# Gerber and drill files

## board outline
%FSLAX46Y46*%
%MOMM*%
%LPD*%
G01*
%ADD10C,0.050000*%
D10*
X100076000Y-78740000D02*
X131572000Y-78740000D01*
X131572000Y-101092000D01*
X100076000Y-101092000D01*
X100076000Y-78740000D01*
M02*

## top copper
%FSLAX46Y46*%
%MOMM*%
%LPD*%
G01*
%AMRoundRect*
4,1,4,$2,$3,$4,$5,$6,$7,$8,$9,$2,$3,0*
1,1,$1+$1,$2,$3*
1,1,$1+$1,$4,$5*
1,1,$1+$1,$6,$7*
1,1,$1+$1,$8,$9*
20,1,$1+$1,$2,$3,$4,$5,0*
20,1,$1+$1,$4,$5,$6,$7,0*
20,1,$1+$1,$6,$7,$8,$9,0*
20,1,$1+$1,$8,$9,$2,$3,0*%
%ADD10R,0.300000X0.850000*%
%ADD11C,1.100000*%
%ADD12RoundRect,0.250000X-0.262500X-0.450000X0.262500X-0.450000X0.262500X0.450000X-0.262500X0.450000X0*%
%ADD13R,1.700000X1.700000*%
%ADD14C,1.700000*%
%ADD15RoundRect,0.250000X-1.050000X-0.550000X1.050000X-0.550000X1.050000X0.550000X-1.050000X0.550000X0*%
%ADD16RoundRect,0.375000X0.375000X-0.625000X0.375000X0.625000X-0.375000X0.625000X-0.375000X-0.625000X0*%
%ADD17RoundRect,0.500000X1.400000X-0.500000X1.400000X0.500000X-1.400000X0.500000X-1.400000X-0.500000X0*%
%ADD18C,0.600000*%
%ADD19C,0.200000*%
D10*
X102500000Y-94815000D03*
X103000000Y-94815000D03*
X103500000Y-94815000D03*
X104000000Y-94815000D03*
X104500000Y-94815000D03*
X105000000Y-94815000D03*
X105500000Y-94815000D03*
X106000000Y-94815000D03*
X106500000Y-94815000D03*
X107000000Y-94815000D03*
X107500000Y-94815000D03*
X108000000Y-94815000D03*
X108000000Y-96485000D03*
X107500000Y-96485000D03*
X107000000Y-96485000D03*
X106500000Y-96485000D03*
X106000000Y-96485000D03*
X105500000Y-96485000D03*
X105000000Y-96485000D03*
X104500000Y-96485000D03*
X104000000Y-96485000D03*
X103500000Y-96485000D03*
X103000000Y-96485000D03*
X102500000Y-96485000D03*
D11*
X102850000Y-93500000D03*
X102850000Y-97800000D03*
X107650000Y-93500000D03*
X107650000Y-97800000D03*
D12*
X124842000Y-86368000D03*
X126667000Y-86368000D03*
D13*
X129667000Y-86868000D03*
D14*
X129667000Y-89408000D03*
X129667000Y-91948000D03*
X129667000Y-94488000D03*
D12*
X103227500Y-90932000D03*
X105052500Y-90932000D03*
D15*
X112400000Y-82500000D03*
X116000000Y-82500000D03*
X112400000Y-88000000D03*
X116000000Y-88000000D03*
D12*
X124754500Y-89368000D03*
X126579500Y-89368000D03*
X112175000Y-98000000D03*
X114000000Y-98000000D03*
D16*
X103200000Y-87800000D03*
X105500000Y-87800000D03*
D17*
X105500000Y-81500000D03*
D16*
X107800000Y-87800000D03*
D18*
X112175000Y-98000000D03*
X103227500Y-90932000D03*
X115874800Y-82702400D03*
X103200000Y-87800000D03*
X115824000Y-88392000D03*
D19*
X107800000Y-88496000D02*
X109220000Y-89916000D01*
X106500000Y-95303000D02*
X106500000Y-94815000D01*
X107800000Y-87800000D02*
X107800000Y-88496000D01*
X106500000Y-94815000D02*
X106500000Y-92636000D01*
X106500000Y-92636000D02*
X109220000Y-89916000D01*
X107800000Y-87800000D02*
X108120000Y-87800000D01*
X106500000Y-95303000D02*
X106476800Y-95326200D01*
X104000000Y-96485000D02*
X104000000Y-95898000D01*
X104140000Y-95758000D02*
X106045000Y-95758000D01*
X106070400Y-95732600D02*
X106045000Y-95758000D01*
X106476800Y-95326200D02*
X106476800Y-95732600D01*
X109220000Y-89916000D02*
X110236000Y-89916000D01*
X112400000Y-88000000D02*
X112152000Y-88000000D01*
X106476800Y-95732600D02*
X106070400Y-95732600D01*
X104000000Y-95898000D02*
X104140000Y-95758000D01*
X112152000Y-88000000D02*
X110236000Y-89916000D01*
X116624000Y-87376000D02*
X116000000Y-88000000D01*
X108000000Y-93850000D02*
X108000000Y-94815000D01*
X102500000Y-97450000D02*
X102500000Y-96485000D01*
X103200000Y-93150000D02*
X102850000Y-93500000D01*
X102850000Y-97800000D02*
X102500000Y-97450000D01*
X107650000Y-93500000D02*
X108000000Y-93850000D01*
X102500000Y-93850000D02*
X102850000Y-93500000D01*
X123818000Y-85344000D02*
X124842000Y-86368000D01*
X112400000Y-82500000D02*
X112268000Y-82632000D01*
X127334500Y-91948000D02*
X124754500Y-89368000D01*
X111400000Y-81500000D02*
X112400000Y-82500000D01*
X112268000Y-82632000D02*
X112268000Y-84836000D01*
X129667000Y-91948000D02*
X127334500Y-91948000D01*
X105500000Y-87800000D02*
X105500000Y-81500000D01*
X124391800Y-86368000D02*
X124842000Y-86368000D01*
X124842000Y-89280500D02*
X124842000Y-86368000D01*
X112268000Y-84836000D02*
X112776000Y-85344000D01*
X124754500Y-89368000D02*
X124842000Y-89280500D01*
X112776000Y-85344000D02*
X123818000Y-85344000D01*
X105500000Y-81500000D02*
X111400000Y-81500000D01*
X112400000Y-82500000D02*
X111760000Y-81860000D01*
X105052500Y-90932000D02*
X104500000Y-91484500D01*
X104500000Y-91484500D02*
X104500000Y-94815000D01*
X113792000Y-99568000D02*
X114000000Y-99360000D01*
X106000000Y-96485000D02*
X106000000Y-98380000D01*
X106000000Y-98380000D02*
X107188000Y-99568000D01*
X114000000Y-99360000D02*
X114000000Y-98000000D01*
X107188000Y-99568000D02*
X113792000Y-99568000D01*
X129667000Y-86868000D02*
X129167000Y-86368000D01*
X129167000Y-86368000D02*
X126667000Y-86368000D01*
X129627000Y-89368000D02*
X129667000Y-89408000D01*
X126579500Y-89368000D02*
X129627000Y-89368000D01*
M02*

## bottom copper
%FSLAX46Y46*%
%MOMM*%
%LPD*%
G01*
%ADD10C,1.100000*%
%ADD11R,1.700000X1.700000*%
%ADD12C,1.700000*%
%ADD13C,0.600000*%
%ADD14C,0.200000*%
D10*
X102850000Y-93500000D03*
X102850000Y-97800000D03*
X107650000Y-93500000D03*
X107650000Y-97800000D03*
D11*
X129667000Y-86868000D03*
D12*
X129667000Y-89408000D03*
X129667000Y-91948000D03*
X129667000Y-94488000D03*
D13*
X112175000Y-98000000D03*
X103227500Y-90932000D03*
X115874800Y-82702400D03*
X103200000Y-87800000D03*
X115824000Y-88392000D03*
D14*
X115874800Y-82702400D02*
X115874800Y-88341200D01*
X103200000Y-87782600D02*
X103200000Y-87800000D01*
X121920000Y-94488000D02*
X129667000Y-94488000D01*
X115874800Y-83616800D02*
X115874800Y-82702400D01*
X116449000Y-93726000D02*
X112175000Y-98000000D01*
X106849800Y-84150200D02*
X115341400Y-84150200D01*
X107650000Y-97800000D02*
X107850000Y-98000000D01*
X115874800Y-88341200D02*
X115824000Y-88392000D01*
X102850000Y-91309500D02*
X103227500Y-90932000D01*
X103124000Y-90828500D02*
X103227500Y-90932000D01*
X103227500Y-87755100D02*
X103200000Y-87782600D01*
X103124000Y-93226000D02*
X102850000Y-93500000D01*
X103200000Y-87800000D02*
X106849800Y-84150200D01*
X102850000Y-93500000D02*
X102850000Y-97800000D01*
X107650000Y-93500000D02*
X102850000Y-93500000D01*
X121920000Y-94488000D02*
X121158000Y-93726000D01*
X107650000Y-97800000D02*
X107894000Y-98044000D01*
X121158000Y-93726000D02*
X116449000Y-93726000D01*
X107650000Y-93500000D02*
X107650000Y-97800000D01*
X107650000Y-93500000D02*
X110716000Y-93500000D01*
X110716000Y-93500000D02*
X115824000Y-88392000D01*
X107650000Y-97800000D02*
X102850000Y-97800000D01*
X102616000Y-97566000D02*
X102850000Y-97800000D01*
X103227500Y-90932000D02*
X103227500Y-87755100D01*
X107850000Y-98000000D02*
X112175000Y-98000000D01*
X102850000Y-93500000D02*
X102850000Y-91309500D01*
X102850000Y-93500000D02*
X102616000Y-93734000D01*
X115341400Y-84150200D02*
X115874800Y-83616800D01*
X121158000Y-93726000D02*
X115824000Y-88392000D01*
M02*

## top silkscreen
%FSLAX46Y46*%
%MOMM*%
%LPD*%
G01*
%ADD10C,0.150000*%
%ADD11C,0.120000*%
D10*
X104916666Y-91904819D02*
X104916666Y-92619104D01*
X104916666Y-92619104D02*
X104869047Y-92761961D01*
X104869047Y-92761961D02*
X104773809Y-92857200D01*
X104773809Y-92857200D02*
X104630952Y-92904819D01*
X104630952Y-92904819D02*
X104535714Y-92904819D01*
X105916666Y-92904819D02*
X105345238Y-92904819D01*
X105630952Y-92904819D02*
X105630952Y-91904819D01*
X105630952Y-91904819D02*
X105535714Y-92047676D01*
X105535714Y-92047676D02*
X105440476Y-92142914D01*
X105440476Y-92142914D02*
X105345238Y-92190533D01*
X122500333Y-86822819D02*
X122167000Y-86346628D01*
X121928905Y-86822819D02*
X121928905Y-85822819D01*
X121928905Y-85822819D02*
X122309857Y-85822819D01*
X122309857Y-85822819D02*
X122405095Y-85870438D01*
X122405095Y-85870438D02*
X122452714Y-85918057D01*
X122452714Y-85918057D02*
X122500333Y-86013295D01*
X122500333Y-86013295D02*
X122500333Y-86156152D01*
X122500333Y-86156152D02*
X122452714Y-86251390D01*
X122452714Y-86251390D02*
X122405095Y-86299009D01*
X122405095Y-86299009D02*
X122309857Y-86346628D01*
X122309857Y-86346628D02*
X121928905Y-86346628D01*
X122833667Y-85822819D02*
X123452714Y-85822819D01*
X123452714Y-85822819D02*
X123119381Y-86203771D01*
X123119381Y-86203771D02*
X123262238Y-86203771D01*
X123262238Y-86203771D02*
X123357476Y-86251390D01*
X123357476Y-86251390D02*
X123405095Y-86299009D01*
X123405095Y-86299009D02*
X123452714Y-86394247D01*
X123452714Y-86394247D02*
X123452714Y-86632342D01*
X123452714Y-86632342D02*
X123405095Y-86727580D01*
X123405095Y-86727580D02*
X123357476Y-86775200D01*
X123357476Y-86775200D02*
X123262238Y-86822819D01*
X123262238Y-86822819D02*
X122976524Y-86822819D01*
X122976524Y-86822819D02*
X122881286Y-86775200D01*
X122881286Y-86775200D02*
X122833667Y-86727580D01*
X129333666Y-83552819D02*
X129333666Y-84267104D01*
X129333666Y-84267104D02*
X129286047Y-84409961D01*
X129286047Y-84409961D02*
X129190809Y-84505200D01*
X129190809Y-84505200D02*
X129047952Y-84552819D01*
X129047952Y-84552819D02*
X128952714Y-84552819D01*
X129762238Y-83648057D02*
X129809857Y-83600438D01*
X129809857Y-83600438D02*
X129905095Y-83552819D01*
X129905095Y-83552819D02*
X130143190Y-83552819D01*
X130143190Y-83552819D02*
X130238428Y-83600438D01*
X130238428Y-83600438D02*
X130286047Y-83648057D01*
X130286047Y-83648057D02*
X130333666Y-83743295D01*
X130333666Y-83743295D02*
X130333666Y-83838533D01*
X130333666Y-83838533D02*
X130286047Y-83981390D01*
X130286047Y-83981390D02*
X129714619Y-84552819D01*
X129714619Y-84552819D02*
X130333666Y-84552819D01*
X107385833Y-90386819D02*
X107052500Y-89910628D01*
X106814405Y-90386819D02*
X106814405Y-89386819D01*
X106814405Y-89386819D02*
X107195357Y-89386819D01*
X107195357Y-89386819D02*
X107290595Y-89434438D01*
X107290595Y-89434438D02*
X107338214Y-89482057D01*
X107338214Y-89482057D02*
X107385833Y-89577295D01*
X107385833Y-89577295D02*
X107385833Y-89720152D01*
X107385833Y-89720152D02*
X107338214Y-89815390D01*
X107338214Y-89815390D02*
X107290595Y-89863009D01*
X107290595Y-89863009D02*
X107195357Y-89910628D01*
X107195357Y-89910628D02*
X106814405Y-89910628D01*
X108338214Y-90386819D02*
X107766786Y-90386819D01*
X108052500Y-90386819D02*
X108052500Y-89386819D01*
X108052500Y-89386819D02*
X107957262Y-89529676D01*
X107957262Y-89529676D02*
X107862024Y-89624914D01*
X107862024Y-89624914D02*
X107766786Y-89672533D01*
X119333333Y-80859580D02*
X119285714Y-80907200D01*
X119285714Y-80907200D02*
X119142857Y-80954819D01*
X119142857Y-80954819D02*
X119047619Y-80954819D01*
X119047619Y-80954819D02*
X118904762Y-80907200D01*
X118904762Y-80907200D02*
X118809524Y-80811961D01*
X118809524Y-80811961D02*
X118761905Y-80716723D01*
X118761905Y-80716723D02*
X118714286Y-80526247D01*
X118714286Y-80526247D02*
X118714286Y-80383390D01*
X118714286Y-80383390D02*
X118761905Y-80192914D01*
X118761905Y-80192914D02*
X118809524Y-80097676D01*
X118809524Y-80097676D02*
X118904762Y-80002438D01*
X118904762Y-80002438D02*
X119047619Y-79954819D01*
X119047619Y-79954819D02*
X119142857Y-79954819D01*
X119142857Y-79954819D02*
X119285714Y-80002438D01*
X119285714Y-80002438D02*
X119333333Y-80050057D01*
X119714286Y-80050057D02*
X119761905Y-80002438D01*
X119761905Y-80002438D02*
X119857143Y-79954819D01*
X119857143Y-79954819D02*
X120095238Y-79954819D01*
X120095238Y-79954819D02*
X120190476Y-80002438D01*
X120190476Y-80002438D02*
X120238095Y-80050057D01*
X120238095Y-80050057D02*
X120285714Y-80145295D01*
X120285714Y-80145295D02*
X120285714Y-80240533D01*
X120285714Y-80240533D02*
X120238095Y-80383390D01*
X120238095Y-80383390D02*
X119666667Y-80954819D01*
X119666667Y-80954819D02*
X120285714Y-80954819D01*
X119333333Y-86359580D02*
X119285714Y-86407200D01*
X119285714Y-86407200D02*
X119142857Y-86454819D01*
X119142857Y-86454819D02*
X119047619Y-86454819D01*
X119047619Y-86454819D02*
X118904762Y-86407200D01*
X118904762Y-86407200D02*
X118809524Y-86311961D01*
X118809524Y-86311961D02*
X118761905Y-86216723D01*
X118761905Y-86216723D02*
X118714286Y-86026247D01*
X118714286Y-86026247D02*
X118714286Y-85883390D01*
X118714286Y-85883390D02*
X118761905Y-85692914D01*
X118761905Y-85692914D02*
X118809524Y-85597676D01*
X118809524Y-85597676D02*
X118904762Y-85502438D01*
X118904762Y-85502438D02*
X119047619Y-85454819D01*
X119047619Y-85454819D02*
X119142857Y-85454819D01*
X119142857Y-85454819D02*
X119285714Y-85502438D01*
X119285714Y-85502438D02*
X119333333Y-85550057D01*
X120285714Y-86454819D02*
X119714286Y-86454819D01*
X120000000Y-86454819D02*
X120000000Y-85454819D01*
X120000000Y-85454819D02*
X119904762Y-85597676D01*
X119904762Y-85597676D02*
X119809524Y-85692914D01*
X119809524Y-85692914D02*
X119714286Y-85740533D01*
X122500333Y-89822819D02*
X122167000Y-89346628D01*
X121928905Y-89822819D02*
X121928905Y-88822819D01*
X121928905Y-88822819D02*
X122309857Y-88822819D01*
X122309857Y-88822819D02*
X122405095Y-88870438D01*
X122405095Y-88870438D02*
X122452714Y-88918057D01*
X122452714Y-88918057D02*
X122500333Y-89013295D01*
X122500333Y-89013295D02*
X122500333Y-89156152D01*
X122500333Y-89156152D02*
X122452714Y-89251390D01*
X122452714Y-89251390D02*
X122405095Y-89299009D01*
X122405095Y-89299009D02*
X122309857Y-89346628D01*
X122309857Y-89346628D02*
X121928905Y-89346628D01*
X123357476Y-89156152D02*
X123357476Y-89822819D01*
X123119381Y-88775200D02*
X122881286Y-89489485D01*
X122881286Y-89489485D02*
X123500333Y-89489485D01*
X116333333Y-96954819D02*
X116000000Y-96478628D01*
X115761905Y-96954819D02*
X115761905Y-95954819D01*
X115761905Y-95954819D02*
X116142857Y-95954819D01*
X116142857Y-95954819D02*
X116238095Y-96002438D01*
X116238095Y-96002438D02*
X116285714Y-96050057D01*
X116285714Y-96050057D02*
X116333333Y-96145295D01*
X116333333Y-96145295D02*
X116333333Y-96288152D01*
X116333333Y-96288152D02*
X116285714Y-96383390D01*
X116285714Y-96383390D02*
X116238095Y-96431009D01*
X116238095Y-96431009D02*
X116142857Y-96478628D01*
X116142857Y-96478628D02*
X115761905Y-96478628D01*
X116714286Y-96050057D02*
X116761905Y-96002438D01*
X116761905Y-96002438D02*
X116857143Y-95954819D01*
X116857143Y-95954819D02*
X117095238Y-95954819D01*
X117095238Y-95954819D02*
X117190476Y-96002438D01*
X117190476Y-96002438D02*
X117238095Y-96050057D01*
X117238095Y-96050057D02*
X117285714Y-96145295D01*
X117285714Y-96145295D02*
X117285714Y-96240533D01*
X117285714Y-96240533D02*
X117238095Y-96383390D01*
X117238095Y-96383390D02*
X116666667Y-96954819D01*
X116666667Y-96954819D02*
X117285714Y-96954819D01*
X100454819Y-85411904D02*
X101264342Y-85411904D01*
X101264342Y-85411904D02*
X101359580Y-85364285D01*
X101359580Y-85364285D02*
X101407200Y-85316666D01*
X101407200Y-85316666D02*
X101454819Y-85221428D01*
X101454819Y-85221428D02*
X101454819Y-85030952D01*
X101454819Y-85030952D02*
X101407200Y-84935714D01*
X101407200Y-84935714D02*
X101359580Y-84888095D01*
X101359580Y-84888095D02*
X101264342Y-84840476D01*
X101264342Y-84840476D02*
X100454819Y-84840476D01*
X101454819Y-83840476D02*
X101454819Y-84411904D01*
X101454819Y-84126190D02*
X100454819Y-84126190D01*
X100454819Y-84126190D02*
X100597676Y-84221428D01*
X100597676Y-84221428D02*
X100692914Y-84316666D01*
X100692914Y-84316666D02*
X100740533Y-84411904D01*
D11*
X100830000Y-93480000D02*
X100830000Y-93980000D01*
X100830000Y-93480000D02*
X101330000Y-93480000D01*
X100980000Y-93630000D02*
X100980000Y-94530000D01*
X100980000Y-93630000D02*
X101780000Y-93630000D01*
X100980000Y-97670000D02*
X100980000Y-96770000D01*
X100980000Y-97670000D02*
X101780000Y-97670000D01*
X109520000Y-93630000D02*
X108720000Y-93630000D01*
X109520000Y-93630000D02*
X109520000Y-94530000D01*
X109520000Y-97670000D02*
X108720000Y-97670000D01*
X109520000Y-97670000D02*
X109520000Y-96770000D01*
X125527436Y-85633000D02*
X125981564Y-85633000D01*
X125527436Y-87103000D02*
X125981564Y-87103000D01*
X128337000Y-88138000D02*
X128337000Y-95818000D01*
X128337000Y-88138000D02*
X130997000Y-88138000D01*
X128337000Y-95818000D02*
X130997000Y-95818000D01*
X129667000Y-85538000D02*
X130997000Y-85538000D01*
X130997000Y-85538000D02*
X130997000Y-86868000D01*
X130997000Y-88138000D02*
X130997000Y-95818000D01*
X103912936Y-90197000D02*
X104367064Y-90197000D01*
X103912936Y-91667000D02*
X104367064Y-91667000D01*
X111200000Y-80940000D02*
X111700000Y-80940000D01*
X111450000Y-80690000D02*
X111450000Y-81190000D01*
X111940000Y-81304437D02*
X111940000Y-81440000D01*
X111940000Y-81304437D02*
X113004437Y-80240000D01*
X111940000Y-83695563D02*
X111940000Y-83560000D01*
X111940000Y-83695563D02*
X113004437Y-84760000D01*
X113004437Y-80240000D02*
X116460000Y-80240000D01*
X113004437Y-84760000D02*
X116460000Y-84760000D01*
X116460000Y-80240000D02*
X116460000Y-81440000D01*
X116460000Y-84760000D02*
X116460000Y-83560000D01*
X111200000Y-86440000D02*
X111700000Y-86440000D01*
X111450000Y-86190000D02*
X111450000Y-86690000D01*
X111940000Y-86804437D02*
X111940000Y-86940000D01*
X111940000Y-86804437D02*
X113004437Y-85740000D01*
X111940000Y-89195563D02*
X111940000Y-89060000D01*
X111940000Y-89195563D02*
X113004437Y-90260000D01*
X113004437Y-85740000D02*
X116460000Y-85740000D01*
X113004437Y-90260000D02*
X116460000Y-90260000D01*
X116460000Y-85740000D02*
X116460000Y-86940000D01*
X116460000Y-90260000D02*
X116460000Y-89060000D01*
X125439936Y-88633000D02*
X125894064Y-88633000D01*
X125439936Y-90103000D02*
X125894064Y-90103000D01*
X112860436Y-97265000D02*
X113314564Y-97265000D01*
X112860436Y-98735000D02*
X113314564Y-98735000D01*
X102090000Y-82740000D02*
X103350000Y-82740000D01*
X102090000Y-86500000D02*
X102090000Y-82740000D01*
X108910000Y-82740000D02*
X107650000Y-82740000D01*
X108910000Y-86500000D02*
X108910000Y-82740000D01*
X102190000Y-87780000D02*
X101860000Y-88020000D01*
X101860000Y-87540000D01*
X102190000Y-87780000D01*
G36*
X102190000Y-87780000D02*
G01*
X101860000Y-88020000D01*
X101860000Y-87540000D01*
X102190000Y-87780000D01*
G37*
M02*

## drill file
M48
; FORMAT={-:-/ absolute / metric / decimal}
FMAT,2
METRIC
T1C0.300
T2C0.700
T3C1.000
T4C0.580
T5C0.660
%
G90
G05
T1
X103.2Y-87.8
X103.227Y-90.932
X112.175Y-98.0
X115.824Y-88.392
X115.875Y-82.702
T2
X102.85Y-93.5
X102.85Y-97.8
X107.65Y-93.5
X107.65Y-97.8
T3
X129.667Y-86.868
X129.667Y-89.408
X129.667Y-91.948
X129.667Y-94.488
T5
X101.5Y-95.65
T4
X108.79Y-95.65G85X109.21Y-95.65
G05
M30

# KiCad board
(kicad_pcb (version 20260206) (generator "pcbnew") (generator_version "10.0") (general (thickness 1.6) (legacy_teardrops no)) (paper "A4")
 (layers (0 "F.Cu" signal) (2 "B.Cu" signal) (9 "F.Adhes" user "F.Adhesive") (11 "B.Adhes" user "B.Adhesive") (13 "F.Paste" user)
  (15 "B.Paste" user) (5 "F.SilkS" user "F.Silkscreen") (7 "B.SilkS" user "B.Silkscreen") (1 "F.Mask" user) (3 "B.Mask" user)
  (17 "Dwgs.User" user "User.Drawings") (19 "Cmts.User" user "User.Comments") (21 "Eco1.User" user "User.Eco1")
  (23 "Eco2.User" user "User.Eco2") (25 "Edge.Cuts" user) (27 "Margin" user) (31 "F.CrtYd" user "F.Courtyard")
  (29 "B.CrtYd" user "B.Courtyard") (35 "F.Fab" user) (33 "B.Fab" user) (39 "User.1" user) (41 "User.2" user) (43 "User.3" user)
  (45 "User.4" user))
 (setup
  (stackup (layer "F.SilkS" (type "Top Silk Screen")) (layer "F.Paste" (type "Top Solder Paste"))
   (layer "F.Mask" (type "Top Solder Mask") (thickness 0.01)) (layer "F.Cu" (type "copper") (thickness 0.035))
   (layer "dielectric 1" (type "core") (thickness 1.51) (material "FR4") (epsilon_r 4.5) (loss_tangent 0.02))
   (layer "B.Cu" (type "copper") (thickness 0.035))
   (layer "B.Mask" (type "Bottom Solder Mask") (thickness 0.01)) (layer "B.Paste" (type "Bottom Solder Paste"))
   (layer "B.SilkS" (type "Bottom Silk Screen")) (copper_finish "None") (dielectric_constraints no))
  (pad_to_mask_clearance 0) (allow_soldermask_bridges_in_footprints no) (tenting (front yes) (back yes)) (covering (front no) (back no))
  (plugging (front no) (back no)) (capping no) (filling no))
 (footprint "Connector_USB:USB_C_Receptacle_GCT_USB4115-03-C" (layer "F.Cu") (at 105.25 95.65)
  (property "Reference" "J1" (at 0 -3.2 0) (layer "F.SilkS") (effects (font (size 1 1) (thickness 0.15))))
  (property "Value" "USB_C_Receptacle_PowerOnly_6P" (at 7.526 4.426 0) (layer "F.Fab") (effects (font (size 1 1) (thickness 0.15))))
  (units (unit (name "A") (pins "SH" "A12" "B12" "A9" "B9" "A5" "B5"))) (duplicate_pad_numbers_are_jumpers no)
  (fp_line (start -4.42 -2.17) (end -4.42 -1.67) (stroke (width 0.12) (type solid)) (layer "F.SilkS"))
  (fp_line (start -4.42 -2.17) (end -3.92 -2.17) (stroke (width 0.12) (type solid)) (layer "F.SilkS"))
  (fp_line (start -4.27 -2.02) (end -4.27 -1.12) (stroke (width 0.12) (type solid)) (layer "F.SilkS"))
  (fp_line (start -4.27 -2.02) (end -3.47 -2.02) (stroke (width 0.12) (type solid)) (layer "F.SilkS"))
  (fp_line (start -4.27 2.02) (end -4.27 1.12) (stroke (width 0.12) (type solid)) (layer "F.SilkS"))
  (fp_line (start -4.27 2.02) (end -3.47 2.02) (stroke (width 0.12) (type solid)) (layer "F.SilkS"))
  (fp_line (start 4.27 -2.02) (end 3.47 -2.02) (stroke (width 0.12) (type solid)) (layer "F.SilkS"))
  (fp_line (start 4.27 -2.02) (end 4.27 -1.12) (stroke (width 0.12) (type solid)) (layer "F.SilkS"))
  (fp_line (start 4.27 2.02) (end 3.47 2.02) (stroke (width 0.12) (type solid)) (layer "F.SilkS"))
  (fp_line (start 4.27 2.02) (end 4.27 1.12) (stroke (width 0.12) (type solid)) (layer "F.SilkS"))
  (pad "" np_thru_hole circle (at -3.75 0) (size 0.66 0.66) (drill 0.66) (layers "*.Cu" "*.Mask"))
  (pad "" np_thru_hole oval (at 3.75 0) (size 1 0.58) (drill oval 1 0.58) (layers "*.Cu" "*.Mask"))
  (pad "A1" smd rect (at -2.75 -0.835) (size 0.3 0.85) (layers "F.Cu" "F.Mask" "F.Paste"))
  (pad "A2" smd rect (at -2.25 -0.835) (size 0.3 0.85) (layers "F.Cu" "F.Mask" "F.Paste"))
  (pad "A3" smd rect (at -1.75 -0.835) (size 0.3 0.85) (layers "F.Cu" "F.Mask" "F.Paste"))
  (pad "A4" smd rect (at -1.25 -0.835) (size 0.3 0.85) (layers "F.Cu" "F.Mask" "F.Paste"))
  (pad "A5" smd rect (at -0.75 -0.835) (size 0.3 0.85) (layers "F.Cu" "F.Mask" "F.Paste") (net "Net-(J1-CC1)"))
  (pad "A6" smd rect (at -0.25 -0.835) (size 0.3 0.85) (layers "F.Cu" "F.Mask" "F.Paste"))
  (pad "A7" smd rect (at 0.25 -0.835) (size 0.3 0.85) (layers "F.Cu" "F.Mask" "F.Paste"))
  (pad "A8" smd rect (at 0.75 -0.835) (size 0.3 0.85) (layers "F.Cu" "F.Mask" "F.Paste"))
  (pad "A9" smd rect (at 1.25 -0.835) (size 0.3 0.85) (layers "F.Cu" "F.Mask" "F.Paste") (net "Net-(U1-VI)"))
  (pad "A10" smd rect (at 1.75 -0.835) (size 0.3 0.85) (layers "F.Cu" "F.Mask" "F.Paste"))
  (pad "A11" smd rect (at 2.25 -0.835) (size 0.3 0.85) (layers "F.Cu" "F.Mask" "F.Paste"))
  (pad "A12" smd rect (at 2.75 -0.835) (size 0.3 0.85) (layers "F.Cu" "F.Mask" "F.Paste") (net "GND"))
  (pad "B1" smd rect (at 2.75 0.835) (size 0.3 0.85) (layers "F.Cu" "F.Mask" "F.Paste"))
  (pad "B2" smd rect (at 2.25 0.835) (size 0.3 0.85) (layers "F.Cu" "F.Mask" "F.Paste"))
  (pad "B3" smd rect (at 1.75 0.835) (size 0.3 0.85) (layers "F.Cu" "F.Mask" "F.Paste"))
  (pad "B4" smd rect (at 1.25 0.835) (size 0.3 0.85) (layers "F.Cu" "F.Mask" "F.Paste"))
  (pad "B5" smd rect (at 0.75 0.835) (size 0.3 0.85) (layers "F.Cu" "F.Mask" "F.Paste") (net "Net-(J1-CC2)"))
  (pad "B6" smd rect (at 0.25 0.835) (size 0.3 0.85) (layers "F.Cu" "F.Mask" "F.Paste"))
  (pad "B7" smd rect (at -0.25 0.835) (size 0.3 0.85) (layers "F.Cu" "F.Mask" "F.Paste"))
  (pad "B8" smd rect (at -0.75 0.835) (size 0.3 0.85) (layers "F.Cu" "F.Mask" "F.Paste"))
  (pad "B9" smd rect (at -1.25 0.835) (size 0.3 0.85) (layers "F.Cu" "F.Mask" "F.Paste") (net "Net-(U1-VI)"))
  (pad "B10" smd rect (at -1.75 0.835) (size 0.3 0.85) (layers "F.Cu" "F.Mask" "F.Paste"))
  (pad "B11" smd rect (at -2.25 0.835) (size 0.3 0.85) (layers "F.Cu" "F.Mask" "F.Paste"))
  (pad "B12" smd rect (at -2.75 0.835) (size 0.3 0.85) (layers "F.Cu" "F.Mask" "F.Paste") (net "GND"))
  (pad "SH" thru_hole circle (at -2.4 -2.15) (size 1.1 1.1) (drill 0.7) (layers "*.Cu" "*.Mask" "F.Paste") (remove_unused_layers no)
   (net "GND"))
  (pad "SH" thru_hole circle (at -2.4 2.15) (size 1.1 1.1) (drill 0.7) (layers "*.Cu" "*.Mask" "F.Paste") (remove_unused_layers no)
   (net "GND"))
  (pad "SH" thru_hole circle (at 2.4 -2.15) (size 1.1 1.1) (drill 0.7) (layers "*.Cu" "*.Mask" "F.Paste") (remove_unused_layers no)
   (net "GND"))
  (pad "SH" thru_hole circle (at 2.4 2.15) (size 1.1 1.1) (drill 0.7) (layers "*.Cu" "*.Mask" "F.Paste") (remove_unused_layers no)
   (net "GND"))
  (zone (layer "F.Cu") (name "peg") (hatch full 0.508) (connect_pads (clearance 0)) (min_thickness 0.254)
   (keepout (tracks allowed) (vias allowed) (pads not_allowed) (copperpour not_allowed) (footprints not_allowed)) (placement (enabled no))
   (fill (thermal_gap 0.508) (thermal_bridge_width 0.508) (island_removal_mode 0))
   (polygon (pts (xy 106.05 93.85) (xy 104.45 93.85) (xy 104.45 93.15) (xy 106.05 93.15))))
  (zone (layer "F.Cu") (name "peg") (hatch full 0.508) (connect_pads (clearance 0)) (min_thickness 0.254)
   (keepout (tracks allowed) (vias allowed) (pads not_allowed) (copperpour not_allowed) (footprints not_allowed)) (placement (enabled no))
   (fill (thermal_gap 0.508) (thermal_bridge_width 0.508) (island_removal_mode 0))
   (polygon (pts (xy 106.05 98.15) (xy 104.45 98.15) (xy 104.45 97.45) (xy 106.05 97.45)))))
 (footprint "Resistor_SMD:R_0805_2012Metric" (layer "F.Cu") (at 125.7545 86.368)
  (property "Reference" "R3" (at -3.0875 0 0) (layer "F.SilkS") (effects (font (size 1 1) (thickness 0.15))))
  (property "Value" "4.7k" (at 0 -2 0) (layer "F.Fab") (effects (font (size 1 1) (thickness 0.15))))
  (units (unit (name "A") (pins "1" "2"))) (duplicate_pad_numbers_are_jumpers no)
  (fp_line (start -0.227064 -0.735) (end 0.227064 -0.735) (stroke (width 0.12) (type solid)) (layer "F.SilkS"))
  (fp_line (start -0.227064 0.735) (end 0.227064 0.735) (stroke (width 0.12) (type solid)) (layer "F.SilkS"))
  (pad "1" smd roundrect (at -0.9125 0) (size 1.025 1.4) (layers "F.Cu" "F.Mask" "F.Paste") (roundrect_rratio 0.243902) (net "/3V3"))
  (pad "2" smd roundrect (at 0.9125 0) (size 1.025 1.4) (layers "F.Cu" "F.Mask" "F.Paste") (roundrect_rratio 0.243902) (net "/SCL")))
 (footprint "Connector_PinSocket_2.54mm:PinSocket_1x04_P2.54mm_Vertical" (layer "F.Cu") (at 129.667 86.868)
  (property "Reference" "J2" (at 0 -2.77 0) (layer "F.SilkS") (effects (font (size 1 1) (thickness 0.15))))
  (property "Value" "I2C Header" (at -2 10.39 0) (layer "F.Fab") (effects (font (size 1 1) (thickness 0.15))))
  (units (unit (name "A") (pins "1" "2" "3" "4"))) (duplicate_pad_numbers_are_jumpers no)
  (fp_line (start -1.33 1.27) (end -1.33 8.95) (stroke (width 0.12) (type solid)) (layer "F.SilkS"))
  (fp_line (start -1.33 1.27) (end 1.33 1.27) (stroke (width 0.12) (type solid)) (layer "F.SilkS"))
  (fp_line (start -1.33 8.95) (end 1.33 8.95) (stroke (width 0.12) (type solid)) (layer "F.SilkS"))
  (fp_line (start 0 -1.33) (end 1.33 -1.33) (stroke (width 0.12) (type solid)) (layer "F.SilkS"))
  (fp_line (start 1.33 -1.33) (end 1.33 0) (stroke (width 0.12) (type solid)) (layer "F.SilkS"))
  (fp_line (start 1.33 1.27) (end 1.33 8.95) (stroke (width 0.12) (type solid)) (layer "F.SilkS"))
  (pad "1" thru_hole rect (at 0 0) (size 1.7 1.7) (drill 1) (layers "*.Cu" "*.Mask") (remove_unused_layers no) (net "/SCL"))
  (pad "2" thru_hole circle (at 0 2.54) (size 1.7 1.7) (drill 1) (layers "*.Cu" "*.Mask") (remove_unused_layers no) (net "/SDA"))
  (pad "3" thru_hole circle (at 0 5.08) (size 1.7 1.7) (drill 1) (layers "*.Cu" "*.Mask") (remove_unused_layers no) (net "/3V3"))
  (pad "4" thru_hole circle (at 0 7.62) (size 1.7 1.7) (drill 1) (layers "*.Cu" "*.Mask") (remove_unused_layers no) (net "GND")))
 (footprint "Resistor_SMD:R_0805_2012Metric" (layer "F.Cu") (at 104.14 90.932)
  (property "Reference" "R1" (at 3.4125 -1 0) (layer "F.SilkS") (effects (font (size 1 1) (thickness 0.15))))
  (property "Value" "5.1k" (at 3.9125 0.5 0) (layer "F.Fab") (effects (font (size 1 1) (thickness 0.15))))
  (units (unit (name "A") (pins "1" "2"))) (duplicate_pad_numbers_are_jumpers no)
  (fp_line (start -0.227064 -0.735) (end 0.227064 -0.735) (stroke (width 0.12) (type solid)) (layer "F.SilkS"))
  (fp_line (start -0.227064 0.735) (end 0.227064 0.735) (stroke (width 0.12) (type solid)) (layer "F.SilkS"))
  (pad "1" smd roundrect (at -0.9125 0) (size 1.025 1.4) (layers "F.Cu" "F.Mask" "F.Paste") (roundrect_rratio 0.243902) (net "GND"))
  (pad "2" smd roundrect (at 0.9125 0) (size 1.025 1.4) (layers "F.Cu" "F.Mask" "F.Paste") (roundrect_rratio 0.243902) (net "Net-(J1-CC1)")))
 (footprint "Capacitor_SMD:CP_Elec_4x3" (layer "F.Cu") (at 114.2 82.5)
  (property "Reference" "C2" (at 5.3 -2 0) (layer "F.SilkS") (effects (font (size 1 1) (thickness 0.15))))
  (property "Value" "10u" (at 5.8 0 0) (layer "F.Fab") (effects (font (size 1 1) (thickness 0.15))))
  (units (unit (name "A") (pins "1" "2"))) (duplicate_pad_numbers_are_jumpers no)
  (fp_line (start -3 -1.56) (end -2.5 -1.56) (stroke (width 0.12) (type solid)) (layer "F.SilkS"))
  (fp_line (start -2.75 -1.81) (end -2.75 -1.31) (stroke (width 0.12) (type solid)) (layer "F.SilkS"))
  (fp_line (start -2.26 -1.195563) (end -2.26 -1.06) (stroke (width 0.12) (type solid)) (layer "F.SilkS"))
  (fp_line (start -2.26 -1.195563) (end -1.195563 -2.26) (stroke (width 0.12) (type solid)) (layer "F.SilkS"))
  (fp_line (start -2.26 1.195563) (end -2.26 1.06) (stroke (width 0.12) (type solid)) (layer "F.SilkS"))
  (fp_line (start -2.26 1.195563) (end -1.195563 2.26) (stroke (width 0.12) (type solid)) (layer "F.SilkS"))
  (fp_line (start -1.195563 -2.26) (end 2.26 -2.26) (stroke (width 0.12) (type solid)) (layer "F.SilkS"))
  (fp_line (start -1.195563 2.26) (end 2.26 2.26) (stroke (width 0.12) (type solid)) (layer "F.SilkS"))
  (fp_line (start 2.26 -2.26) (end 2.26 -1.06) (stroke (width 0.12) (type solid)) (layer "F.SilkS"))
  (fp_line (start 2.26 2.26) (end 2.26 1.06) (stroke (width 0.12) (type solid)) (layer "F.SilkS"))
  (pad "1" smd roundrect (at -1.8 0) (size 2.6 1.6) (layers "F.Cu" "F.Mask" "F.Paste") (roundrect_rratio 0.15625) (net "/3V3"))
  (pad "2" smd roundrect (at 1.8 0) (size 2.6 1.6) (layers "F.Cu" "F.Mask" "F.Paste") (roundrect_rratio 0.15625) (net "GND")))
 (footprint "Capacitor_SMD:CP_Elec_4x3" (layer "F.Cu") (at 114.2 88)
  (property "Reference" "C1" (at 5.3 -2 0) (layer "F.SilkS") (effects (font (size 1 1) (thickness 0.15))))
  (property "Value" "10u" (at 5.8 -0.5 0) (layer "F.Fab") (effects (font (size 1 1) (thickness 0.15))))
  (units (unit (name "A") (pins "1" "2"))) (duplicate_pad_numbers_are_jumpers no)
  (fp_line (start -3 -1.56) (end -2.5 -1.56) (stroke (width 0.12) (type solid)) (layer "F.SilkS"))
  (fp_line (start -2.75 -1.81) (end -2.75 -1.31) (stroke (width 0.12) (type solid)) (layer "F.SilkS"))
  (fp_line (start -2.26 -1.195563) (end -2.26 -1.06) (stroke (width 0.12) (type solid)) (layer "F.SilkS"))
  (fp_line (start -2.26 -1.195563) (end -1.195563 -2.26) (stroke (width 0.12) (type solid)) (layer "F.SilkS"))
  (fp_line (start -2.26 1.195563) (end -2.26 1.06) (stroke (width 0.12) (type solid)) (layer "F.SilkS"))
  (fp_line (start -2.26 1.195563) (end -1.195563 2.26) (stroke (width 0.12) (type solid)) (layer "F.SilkS"))
  (fp_line (start -1.195563 -2.26) (end 2.26 -2.26) (stroke (width 0.12) (type solid)) (layer "F.SilkS"))
  (fp_line (start -1.195563 2.26) (end 2.26 2.26) (stroke (width 0.12) (type solid)) (layer "F.SilkS"))
  (fp_line (start 2.26 -2.26) (end 2.26 -1.06) (stroke (width 0.12) (type solid)) (layer "F.SilkS"))
  (fp_line (start 2.26 2.26) (end 2.26 1.06) (stroke (width 0.12) (type solid)) (layer "F.SilkS"))
  (pad "1" smd roundrect (at -1.8 0) (size 2.6 1.6) (layers "F.Cu" "F.Mask" "F.Paste") (roundrect_rratio 0.15625) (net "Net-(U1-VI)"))
  (pad "2" smd roundrect (at 1.8 0) (size 2.6 1.6) (layers "F.Cu" "F.Mask" "F.Paste") (roundrect_rratio 0.15625) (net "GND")))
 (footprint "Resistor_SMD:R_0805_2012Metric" (layer "F.Cu") (at 125.667 89.368)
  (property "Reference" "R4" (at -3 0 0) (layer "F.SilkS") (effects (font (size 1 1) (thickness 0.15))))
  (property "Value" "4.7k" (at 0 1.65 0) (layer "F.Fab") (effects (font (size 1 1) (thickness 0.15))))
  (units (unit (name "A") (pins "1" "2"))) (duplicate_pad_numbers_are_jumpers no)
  (fp_line (start -0.227064 -0.735) (end 0.227064 -0.735) (stroke (width 0.12) (type solid)) (layer "F.SilkS"))
  (fp_line (start -0.227064 0.735) (end 0.227064 0.735) (stroke (width 0.12) (type solid)) (layer "F.SilkS"))
  (pad "1" smd roundrect (at -0.9125 0) (size 1.025 1.4) (layers "F.Cu" "F.Mask" "F.Paste") (roundrect_rratio 0.243902) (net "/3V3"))
  (pad "2" smd roundrect (at 0.9125 0) (size 1.025 1.4) (layers "F.Cu" "F.Mask" "F.Paste") (roundrect_rratio 0.243902) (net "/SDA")))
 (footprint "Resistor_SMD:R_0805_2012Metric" (layer "F.Cu") (at 113.0875 98)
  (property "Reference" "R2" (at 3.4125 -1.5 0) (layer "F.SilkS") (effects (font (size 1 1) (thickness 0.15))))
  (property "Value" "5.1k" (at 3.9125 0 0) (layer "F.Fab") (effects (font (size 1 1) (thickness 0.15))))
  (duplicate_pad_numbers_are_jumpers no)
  (fp_line (start -0.227064 -0.735) (end 0.227064 -0.735) (stroke (width 0.12) (type solid)) (layer "F.SilkS"))
  (fp_line (start -0.227064 0.735) (end 0.227064 0.735) (stroke (width 0.12) (type solid)) (layer "F.SilkS"))
  (pad "1" smd roundrect (at -0.9125 0) (size 1.025 1.4) (layers "F.Cu" "F.Mask" "F.Paste") (roundrect_rratio 0.243902) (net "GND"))
  (pad "2" smd roundrect (at 0.9125 0) (size 1.025 1.4) (layers "F.Cu" "F.Mask" "F.Paste") (roundrect_rratio 0.243902) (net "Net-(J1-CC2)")))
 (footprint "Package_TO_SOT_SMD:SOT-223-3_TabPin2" (layer "F.Cu") (at 105.5 84.65 90)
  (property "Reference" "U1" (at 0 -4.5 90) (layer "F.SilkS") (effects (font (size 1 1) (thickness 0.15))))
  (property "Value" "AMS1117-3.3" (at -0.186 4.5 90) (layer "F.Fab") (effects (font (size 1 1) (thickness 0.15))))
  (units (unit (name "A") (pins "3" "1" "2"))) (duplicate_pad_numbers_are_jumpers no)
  (fp_line (start 1.91 -3.41) (end 1.91 -2.15) (stroke (width 0.12) (type solid)) (layer "F.SilkS"))
  (fp_line (start -1.85 -3.41) (end 1.91 -3.41) (stroke (width 0.12) (type solid)) (layer "F.SilkS"))
  (fp_line (start 1.91 3.41) (end 1.91 2.15) (stroke (width 0.12) (type solid)) (layer "F.SilkS"))
  (fp_line (start -1.85 3.41) (end 1.91 3.41) (stroke (width 0.12) (type solid)) (layer "F.SilkS"))
  (fp_poly
   (pts (xy -3.13 -3.31) (xy -3.37 -3.64) (xy -2.89 -3.64) (xy -3.13 -3.31)) (stroke (width 0.12) (type solid)) (fill yes) (layer "F.SilkS"))
  (pad "1" smd roundrect (at -3.15 -2.3 90) (size 2 1.5) (layers "F.Cu" "F.Mask" "F.Paste") (roundrect_rratio 0.25) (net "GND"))
  (pad "2" smd roundrect (at -3.15 0 90) (size 2 1.5) (layers "F.Cu" "F.Mask" "F.Paste") (roundrect_rratio 0.25) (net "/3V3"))
  (pad "2" smd roundrect (at 3.15 0 90) (size 2 3.8) (layers "F.Cu" "F.Mask" "F.Paste") (roundrect_rratio 0.25) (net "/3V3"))
  (pad "3" smd roundrect (at -3.15 2.3 90) (size 2 1.5) (layers "F.Cu" "F.Mask" "F.Paste") (roundrect_rratio 0.25) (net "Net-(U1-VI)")))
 (gr_rect (start 100.076 78.74) (end 131.572 101.092) (stroke (width 0.05) (type default)) (fill no) (layer "Edge.Cuts"))
 (segment (start 107.8 88.496) (end 109.22 89.916) (width 0.2) (layer "F.Cu") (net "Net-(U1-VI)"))
 (segment (start 106.5 95.303) (end 106.5 94.815) (width 0.2) (layer "F.Cu") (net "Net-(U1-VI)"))
 (segment (start 107.8 87.8) (end 107.8 88.496) (width 0.2) (layer "F.Cu") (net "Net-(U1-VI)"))
 (segment (start 106.5 94.815) (end 106.5 92.636) (width 0.2) (layer "F.Cu") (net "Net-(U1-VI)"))
 (segment (start 106.5 92.636) (end 109.22 89.916) (width 0.2) (layer "F.Cu") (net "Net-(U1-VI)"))
 (segment (start 107.8 87.8) (end 108.12 87.8) (width 0.2) (layer "F.Cu") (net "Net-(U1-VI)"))
 (segment (start 106.5 95.303) (end 106.4768 95.3262) (width 0.2) (layer "F.Cu") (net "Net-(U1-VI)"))
 (segment (start 104 96.485) (end 104 95.898) (width 0.2) (layer "F.Cu") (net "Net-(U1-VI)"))
 (segment (start 104.14 95.758) (end 106.045 95.758) (width 0.2) (layer "F.Cu") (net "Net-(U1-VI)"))
 (segment (start 106.0704 95.7326) (end 106.045 95.758) (width 0.2) (layer "F.Cu") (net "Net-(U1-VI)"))
 (segment (start 106.4768 95.3262) (end 106.4768 95.7326) (width 0.2) (layer "F.Cu") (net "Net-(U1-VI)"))
 (segment (start 109.22 89.916) (end 110.236 89.916) (width 0.2) (layer "F.Cu") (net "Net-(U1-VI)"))
 (segment (start 112.4 88) (end 112.152 88) (width 0.2) (layer "F.Cu") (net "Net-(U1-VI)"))
 (segment (start 106.4768 95.7326) (end 106.0704 95.7326) (width 0.2) (layer "F.Cu") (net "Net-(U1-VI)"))
 (segment (start 104 95.898) (end 104.14 95.758) (width 0.2) (layer "F.Cu") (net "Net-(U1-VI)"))
 (segment (start 112.152 88) (end 110.236 89.916) (width 0.2) (layer "F.Cu") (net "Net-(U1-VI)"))
 (segment (start 116.624 87.376) (end 116 88) (width 0.2) (layer "F.Cu") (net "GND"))
 (segment (start 108 93.85) (end 108 94.815) (width 0.2) (layer "F.Cu") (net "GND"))
 (segment (start 102.5 97.45) (end 102.5 96.485) (width 0.2) (layer "F.Cu") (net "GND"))
 (segment (start 103.2 93.15) (end 102.85 93.5) (width 0.2) (layer "F.Cu") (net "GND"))
 (segment (start 102.85 97.8) (end 102.5 97.45) (width 0.2) (layer "F.Cu") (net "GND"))
 (segment (start 107.65 93.5) (end 108 93.85) (width 0.2) (layer "F.Cu") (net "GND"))
 (segment (start 102.5 93.85) (end 102.85 93.5) (width 0.2) (layer "F.Cu") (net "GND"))
 (via (at 112.175 98) (size 0.6) (drill 0.3) (layers "F.Cu" "B.Cu") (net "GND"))
 (via (at 103.2275 90.932) (size 0.6) (drill 0.3) (layers "F.Cu" "B.Cu") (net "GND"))
 (via (at 115.8748 82.7024) (size 0.6) (drill 0.3) (layers "F.Cu" "B.Cu") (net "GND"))
 (via (at 103.2 87.8) (size 0.6) (drill 0.3) (layers "F.Cu" "B.Cu") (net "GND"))
 (via (at 115.824 88.392) (size 0.6) (drill 0.3) (layers "F.Cu" "B.Cu") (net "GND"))
 (segment (start 115.8748 82.7024) (end 115.8748 88.3412) (width 0.2) (layer "B.Cu") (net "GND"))
 (segment (start 103.2 87.7826) (end 103.2 87.8) (width 0.2) (layer "B.Cu") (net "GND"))
 (segment (start 121.92 94.488) (end 129.667 94.488) (width 0.2) (layer "B.Cu") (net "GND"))
 (segment (start 115.8748 83.6168) (end 115.8748 82.7024) (width 0.2) (layer "B.Cu") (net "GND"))
 (segment (start 116.449 93.726) (end 112.175 98) (width 0.2) (layer "B.Cu") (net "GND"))
 (segment (start 106.8498 84.1502) (end 115.3414 84.1502) (width 0.2) (layer "B.Cu") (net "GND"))
 (segment (start 107.65 97.8) (end 107.85 98) (width 0.2) (layer "B.Cu") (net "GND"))
 (segment (start 115.8748 88.3412) (end 115.824 88.392) (width 0.2) (layer "B.Cu") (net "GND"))
 (segment (start 102.85 91.3095) (end 103.2275 90.932) (width 0.2) (layer "B.Cu") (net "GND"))
 (segment (start 103.124 90.8285) (end 103.2275 90.932) (width 0.2) (layer "B.Cu") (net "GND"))
 (segment (start 103.2275 87.7551) (end 103.2 87.7826) (width 0.2) (layer "B.Cu") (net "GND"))
 (segment (start 103.124 93.226) (end 102.85 93.5) (width 0.2) (layer "B.Cu") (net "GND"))
 (segment (start 103.2 87.8) (end 106.8498 84.1502) (width 0.2) (layer "B.Cu") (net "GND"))
 (segment (start 102.85 93.5) (end 102.85 97.8) (width 0.2) (layer "B.Cu") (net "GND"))
 (segment (start 107.65 93.5) (end 102.85 93.5) (width 0.2) (layer "B.Cu") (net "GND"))
 (segment (start 121.92 94.488) (end 121.158 93.726) (width 0.2) (layer "B.Cu") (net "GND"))
 (segment (start 107.65 97.8) (end 107.894 98.044) (width 0.2) (layer "B.Cu") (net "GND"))
 (segment (start 121.158 93.726) (end 116.449 93.726) (width 0.2) (layer "B.Cu") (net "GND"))
 (segment (start 107.65 93.5) (end 107.65 97.8) (width 0.2) (layer "B.Cu") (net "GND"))
 (segment (start 107.65 93.5) (end 110.716 93.5) (width 0.2) (layer "B.Cu") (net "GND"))
 (segment (start 110.716 93.5) (end 115.824 88.392) (width 0.2) (layer "B.Cu") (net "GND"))
 (segment (start 107.65 97.8) (end 102.85 97.8) (width 0.2) (layer "B.Cu") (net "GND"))
 (segment (start 102.616 97.566) (end 102.85 97.8) (width 0.2) (layer "B.Cu") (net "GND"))
 (segment (start 103.2275 90.932) (end 103.2275 87.7551) (width 0.2) (layer "B.Cu") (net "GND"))
 (segment (start 107.85 98) (end 112.175 98) (width 0.2) (layer "B.Cu") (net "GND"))
 (segment (start 102.85 93.5) (end 102.85 91.3095) (width 0.2) (layer "B.Cu") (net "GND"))
 (segment (start 102.85 93.5) (end 102.616 93.734) (width 0.2) (layer "B.Cu") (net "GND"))
 (segment (start 115.3414 84.1502) (end 115.8748 83.6168) (width 0.2) (layer "B.Cu") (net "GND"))
 (segment (start 121.158 93.726) (end 115.824 88.392) (width 0.2) (layer "B.Cu") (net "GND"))
 (segment (start 123.818 85.344) (end 124.842 86.368) (width 0.2) (layer "F.Cu") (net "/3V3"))
 (segment (start 112.4 82.5) (end 112.268 82.632) (width 0.2) (layer "F.Cu") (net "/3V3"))
 (segment (start 127.3345 91.948) (end 124.7545 89.368) (width 0.2) (layer "F.Cu") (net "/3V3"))
 (segment (start 111.4 81.5) (end 112.4 82.5) (width 0.2) (layer "F.Cu") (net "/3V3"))
 (segment (start 112.268 82.632) (end 112.268 84.836) (width 0.2) (layer "F.Cu") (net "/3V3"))
 (segment (start 129.667 91.948) (end 127.3345 91.948) (width 0.2) (layer "F.Cu") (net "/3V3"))
 (segment (start 105.5 87.8) (end 105.5 81.5) (width 0.2) (layer "F.Cu") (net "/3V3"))
 (segment (start 124.3918 86.368) (end 124.842 86.368) (width 0.2) (layer "F.Cu") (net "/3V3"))
 (segment (start 124.842 89.2805) (end 124.842 86.368) (width 0.2) (layer "F.Cu") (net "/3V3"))
 (segment (start 112.268 84.836) (end 112.776 85.344) (width 0.2) (layer "F.Cu") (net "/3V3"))
 (segment (start 124.7545 89.368) (end 124.842 89.2805) (width 0.2) (layer "F.Cu") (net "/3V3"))
 (segment (start 112.776 85.344) (end 123.818 85.344) (width 0.2) (layer "F.Cu") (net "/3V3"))
 (segment (start 105.5 81.5) (end 111.4 81.5) (width 0.2) (layer "F.Cu") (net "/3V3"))
 (segment (start 112.4 82.5) (end 111.76 81.86) (width 0.2) (layer "F.Cu") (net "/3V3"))
 (segment (start 105.0525 90.932) (end 104.5 91.4845) (width 0.2) (layer "F.Cu") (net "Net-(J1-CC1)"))
 (segment (start 104.5 91.4845) (end 104.5 94.815) (width 0.2) (layer "F.Cu") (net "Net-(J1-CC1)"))
 (segment (start 113.792 99.568) (end 114 99.36) (width 0.2) (layer "F.Cu") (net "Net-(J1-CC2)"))
 (segment (start 106 96.485) (end 106 98.38) (width 0.2) (layer "F.Cu") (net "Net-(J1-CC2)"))
 (segment (start 106 98.38) (end 107.188 99.568) (width 0.2) (layer "F.Cu") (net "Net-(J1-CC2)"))
 (segment (start 114 99.36) (end 114 98) (width 0.2) (layer "F.Cu") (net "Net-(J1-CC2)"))
 (segment (start 107.188 99.568) (end 113.792 99.568) (width 0.2) (layer "F.Cu") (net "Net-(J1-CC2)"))
 (segment (start 129.667 86.868) (end 129.167 86.368) (width 0.2) (layer "F.Cu") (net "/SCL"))
 (segment (start 129.167 86.368) (end 126.667 86.368) (width 0.2) (layer "F.Cu") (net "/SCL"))
 (segment (start 129.627 89.368) (end 129.667 89.408) (width 0.2) (layer "F.Cu") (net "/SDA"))
 (segment (start 126.5795 89.368) (end 129.627 89.368) (width 0.2) (layer "F.Cu") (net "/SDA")))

